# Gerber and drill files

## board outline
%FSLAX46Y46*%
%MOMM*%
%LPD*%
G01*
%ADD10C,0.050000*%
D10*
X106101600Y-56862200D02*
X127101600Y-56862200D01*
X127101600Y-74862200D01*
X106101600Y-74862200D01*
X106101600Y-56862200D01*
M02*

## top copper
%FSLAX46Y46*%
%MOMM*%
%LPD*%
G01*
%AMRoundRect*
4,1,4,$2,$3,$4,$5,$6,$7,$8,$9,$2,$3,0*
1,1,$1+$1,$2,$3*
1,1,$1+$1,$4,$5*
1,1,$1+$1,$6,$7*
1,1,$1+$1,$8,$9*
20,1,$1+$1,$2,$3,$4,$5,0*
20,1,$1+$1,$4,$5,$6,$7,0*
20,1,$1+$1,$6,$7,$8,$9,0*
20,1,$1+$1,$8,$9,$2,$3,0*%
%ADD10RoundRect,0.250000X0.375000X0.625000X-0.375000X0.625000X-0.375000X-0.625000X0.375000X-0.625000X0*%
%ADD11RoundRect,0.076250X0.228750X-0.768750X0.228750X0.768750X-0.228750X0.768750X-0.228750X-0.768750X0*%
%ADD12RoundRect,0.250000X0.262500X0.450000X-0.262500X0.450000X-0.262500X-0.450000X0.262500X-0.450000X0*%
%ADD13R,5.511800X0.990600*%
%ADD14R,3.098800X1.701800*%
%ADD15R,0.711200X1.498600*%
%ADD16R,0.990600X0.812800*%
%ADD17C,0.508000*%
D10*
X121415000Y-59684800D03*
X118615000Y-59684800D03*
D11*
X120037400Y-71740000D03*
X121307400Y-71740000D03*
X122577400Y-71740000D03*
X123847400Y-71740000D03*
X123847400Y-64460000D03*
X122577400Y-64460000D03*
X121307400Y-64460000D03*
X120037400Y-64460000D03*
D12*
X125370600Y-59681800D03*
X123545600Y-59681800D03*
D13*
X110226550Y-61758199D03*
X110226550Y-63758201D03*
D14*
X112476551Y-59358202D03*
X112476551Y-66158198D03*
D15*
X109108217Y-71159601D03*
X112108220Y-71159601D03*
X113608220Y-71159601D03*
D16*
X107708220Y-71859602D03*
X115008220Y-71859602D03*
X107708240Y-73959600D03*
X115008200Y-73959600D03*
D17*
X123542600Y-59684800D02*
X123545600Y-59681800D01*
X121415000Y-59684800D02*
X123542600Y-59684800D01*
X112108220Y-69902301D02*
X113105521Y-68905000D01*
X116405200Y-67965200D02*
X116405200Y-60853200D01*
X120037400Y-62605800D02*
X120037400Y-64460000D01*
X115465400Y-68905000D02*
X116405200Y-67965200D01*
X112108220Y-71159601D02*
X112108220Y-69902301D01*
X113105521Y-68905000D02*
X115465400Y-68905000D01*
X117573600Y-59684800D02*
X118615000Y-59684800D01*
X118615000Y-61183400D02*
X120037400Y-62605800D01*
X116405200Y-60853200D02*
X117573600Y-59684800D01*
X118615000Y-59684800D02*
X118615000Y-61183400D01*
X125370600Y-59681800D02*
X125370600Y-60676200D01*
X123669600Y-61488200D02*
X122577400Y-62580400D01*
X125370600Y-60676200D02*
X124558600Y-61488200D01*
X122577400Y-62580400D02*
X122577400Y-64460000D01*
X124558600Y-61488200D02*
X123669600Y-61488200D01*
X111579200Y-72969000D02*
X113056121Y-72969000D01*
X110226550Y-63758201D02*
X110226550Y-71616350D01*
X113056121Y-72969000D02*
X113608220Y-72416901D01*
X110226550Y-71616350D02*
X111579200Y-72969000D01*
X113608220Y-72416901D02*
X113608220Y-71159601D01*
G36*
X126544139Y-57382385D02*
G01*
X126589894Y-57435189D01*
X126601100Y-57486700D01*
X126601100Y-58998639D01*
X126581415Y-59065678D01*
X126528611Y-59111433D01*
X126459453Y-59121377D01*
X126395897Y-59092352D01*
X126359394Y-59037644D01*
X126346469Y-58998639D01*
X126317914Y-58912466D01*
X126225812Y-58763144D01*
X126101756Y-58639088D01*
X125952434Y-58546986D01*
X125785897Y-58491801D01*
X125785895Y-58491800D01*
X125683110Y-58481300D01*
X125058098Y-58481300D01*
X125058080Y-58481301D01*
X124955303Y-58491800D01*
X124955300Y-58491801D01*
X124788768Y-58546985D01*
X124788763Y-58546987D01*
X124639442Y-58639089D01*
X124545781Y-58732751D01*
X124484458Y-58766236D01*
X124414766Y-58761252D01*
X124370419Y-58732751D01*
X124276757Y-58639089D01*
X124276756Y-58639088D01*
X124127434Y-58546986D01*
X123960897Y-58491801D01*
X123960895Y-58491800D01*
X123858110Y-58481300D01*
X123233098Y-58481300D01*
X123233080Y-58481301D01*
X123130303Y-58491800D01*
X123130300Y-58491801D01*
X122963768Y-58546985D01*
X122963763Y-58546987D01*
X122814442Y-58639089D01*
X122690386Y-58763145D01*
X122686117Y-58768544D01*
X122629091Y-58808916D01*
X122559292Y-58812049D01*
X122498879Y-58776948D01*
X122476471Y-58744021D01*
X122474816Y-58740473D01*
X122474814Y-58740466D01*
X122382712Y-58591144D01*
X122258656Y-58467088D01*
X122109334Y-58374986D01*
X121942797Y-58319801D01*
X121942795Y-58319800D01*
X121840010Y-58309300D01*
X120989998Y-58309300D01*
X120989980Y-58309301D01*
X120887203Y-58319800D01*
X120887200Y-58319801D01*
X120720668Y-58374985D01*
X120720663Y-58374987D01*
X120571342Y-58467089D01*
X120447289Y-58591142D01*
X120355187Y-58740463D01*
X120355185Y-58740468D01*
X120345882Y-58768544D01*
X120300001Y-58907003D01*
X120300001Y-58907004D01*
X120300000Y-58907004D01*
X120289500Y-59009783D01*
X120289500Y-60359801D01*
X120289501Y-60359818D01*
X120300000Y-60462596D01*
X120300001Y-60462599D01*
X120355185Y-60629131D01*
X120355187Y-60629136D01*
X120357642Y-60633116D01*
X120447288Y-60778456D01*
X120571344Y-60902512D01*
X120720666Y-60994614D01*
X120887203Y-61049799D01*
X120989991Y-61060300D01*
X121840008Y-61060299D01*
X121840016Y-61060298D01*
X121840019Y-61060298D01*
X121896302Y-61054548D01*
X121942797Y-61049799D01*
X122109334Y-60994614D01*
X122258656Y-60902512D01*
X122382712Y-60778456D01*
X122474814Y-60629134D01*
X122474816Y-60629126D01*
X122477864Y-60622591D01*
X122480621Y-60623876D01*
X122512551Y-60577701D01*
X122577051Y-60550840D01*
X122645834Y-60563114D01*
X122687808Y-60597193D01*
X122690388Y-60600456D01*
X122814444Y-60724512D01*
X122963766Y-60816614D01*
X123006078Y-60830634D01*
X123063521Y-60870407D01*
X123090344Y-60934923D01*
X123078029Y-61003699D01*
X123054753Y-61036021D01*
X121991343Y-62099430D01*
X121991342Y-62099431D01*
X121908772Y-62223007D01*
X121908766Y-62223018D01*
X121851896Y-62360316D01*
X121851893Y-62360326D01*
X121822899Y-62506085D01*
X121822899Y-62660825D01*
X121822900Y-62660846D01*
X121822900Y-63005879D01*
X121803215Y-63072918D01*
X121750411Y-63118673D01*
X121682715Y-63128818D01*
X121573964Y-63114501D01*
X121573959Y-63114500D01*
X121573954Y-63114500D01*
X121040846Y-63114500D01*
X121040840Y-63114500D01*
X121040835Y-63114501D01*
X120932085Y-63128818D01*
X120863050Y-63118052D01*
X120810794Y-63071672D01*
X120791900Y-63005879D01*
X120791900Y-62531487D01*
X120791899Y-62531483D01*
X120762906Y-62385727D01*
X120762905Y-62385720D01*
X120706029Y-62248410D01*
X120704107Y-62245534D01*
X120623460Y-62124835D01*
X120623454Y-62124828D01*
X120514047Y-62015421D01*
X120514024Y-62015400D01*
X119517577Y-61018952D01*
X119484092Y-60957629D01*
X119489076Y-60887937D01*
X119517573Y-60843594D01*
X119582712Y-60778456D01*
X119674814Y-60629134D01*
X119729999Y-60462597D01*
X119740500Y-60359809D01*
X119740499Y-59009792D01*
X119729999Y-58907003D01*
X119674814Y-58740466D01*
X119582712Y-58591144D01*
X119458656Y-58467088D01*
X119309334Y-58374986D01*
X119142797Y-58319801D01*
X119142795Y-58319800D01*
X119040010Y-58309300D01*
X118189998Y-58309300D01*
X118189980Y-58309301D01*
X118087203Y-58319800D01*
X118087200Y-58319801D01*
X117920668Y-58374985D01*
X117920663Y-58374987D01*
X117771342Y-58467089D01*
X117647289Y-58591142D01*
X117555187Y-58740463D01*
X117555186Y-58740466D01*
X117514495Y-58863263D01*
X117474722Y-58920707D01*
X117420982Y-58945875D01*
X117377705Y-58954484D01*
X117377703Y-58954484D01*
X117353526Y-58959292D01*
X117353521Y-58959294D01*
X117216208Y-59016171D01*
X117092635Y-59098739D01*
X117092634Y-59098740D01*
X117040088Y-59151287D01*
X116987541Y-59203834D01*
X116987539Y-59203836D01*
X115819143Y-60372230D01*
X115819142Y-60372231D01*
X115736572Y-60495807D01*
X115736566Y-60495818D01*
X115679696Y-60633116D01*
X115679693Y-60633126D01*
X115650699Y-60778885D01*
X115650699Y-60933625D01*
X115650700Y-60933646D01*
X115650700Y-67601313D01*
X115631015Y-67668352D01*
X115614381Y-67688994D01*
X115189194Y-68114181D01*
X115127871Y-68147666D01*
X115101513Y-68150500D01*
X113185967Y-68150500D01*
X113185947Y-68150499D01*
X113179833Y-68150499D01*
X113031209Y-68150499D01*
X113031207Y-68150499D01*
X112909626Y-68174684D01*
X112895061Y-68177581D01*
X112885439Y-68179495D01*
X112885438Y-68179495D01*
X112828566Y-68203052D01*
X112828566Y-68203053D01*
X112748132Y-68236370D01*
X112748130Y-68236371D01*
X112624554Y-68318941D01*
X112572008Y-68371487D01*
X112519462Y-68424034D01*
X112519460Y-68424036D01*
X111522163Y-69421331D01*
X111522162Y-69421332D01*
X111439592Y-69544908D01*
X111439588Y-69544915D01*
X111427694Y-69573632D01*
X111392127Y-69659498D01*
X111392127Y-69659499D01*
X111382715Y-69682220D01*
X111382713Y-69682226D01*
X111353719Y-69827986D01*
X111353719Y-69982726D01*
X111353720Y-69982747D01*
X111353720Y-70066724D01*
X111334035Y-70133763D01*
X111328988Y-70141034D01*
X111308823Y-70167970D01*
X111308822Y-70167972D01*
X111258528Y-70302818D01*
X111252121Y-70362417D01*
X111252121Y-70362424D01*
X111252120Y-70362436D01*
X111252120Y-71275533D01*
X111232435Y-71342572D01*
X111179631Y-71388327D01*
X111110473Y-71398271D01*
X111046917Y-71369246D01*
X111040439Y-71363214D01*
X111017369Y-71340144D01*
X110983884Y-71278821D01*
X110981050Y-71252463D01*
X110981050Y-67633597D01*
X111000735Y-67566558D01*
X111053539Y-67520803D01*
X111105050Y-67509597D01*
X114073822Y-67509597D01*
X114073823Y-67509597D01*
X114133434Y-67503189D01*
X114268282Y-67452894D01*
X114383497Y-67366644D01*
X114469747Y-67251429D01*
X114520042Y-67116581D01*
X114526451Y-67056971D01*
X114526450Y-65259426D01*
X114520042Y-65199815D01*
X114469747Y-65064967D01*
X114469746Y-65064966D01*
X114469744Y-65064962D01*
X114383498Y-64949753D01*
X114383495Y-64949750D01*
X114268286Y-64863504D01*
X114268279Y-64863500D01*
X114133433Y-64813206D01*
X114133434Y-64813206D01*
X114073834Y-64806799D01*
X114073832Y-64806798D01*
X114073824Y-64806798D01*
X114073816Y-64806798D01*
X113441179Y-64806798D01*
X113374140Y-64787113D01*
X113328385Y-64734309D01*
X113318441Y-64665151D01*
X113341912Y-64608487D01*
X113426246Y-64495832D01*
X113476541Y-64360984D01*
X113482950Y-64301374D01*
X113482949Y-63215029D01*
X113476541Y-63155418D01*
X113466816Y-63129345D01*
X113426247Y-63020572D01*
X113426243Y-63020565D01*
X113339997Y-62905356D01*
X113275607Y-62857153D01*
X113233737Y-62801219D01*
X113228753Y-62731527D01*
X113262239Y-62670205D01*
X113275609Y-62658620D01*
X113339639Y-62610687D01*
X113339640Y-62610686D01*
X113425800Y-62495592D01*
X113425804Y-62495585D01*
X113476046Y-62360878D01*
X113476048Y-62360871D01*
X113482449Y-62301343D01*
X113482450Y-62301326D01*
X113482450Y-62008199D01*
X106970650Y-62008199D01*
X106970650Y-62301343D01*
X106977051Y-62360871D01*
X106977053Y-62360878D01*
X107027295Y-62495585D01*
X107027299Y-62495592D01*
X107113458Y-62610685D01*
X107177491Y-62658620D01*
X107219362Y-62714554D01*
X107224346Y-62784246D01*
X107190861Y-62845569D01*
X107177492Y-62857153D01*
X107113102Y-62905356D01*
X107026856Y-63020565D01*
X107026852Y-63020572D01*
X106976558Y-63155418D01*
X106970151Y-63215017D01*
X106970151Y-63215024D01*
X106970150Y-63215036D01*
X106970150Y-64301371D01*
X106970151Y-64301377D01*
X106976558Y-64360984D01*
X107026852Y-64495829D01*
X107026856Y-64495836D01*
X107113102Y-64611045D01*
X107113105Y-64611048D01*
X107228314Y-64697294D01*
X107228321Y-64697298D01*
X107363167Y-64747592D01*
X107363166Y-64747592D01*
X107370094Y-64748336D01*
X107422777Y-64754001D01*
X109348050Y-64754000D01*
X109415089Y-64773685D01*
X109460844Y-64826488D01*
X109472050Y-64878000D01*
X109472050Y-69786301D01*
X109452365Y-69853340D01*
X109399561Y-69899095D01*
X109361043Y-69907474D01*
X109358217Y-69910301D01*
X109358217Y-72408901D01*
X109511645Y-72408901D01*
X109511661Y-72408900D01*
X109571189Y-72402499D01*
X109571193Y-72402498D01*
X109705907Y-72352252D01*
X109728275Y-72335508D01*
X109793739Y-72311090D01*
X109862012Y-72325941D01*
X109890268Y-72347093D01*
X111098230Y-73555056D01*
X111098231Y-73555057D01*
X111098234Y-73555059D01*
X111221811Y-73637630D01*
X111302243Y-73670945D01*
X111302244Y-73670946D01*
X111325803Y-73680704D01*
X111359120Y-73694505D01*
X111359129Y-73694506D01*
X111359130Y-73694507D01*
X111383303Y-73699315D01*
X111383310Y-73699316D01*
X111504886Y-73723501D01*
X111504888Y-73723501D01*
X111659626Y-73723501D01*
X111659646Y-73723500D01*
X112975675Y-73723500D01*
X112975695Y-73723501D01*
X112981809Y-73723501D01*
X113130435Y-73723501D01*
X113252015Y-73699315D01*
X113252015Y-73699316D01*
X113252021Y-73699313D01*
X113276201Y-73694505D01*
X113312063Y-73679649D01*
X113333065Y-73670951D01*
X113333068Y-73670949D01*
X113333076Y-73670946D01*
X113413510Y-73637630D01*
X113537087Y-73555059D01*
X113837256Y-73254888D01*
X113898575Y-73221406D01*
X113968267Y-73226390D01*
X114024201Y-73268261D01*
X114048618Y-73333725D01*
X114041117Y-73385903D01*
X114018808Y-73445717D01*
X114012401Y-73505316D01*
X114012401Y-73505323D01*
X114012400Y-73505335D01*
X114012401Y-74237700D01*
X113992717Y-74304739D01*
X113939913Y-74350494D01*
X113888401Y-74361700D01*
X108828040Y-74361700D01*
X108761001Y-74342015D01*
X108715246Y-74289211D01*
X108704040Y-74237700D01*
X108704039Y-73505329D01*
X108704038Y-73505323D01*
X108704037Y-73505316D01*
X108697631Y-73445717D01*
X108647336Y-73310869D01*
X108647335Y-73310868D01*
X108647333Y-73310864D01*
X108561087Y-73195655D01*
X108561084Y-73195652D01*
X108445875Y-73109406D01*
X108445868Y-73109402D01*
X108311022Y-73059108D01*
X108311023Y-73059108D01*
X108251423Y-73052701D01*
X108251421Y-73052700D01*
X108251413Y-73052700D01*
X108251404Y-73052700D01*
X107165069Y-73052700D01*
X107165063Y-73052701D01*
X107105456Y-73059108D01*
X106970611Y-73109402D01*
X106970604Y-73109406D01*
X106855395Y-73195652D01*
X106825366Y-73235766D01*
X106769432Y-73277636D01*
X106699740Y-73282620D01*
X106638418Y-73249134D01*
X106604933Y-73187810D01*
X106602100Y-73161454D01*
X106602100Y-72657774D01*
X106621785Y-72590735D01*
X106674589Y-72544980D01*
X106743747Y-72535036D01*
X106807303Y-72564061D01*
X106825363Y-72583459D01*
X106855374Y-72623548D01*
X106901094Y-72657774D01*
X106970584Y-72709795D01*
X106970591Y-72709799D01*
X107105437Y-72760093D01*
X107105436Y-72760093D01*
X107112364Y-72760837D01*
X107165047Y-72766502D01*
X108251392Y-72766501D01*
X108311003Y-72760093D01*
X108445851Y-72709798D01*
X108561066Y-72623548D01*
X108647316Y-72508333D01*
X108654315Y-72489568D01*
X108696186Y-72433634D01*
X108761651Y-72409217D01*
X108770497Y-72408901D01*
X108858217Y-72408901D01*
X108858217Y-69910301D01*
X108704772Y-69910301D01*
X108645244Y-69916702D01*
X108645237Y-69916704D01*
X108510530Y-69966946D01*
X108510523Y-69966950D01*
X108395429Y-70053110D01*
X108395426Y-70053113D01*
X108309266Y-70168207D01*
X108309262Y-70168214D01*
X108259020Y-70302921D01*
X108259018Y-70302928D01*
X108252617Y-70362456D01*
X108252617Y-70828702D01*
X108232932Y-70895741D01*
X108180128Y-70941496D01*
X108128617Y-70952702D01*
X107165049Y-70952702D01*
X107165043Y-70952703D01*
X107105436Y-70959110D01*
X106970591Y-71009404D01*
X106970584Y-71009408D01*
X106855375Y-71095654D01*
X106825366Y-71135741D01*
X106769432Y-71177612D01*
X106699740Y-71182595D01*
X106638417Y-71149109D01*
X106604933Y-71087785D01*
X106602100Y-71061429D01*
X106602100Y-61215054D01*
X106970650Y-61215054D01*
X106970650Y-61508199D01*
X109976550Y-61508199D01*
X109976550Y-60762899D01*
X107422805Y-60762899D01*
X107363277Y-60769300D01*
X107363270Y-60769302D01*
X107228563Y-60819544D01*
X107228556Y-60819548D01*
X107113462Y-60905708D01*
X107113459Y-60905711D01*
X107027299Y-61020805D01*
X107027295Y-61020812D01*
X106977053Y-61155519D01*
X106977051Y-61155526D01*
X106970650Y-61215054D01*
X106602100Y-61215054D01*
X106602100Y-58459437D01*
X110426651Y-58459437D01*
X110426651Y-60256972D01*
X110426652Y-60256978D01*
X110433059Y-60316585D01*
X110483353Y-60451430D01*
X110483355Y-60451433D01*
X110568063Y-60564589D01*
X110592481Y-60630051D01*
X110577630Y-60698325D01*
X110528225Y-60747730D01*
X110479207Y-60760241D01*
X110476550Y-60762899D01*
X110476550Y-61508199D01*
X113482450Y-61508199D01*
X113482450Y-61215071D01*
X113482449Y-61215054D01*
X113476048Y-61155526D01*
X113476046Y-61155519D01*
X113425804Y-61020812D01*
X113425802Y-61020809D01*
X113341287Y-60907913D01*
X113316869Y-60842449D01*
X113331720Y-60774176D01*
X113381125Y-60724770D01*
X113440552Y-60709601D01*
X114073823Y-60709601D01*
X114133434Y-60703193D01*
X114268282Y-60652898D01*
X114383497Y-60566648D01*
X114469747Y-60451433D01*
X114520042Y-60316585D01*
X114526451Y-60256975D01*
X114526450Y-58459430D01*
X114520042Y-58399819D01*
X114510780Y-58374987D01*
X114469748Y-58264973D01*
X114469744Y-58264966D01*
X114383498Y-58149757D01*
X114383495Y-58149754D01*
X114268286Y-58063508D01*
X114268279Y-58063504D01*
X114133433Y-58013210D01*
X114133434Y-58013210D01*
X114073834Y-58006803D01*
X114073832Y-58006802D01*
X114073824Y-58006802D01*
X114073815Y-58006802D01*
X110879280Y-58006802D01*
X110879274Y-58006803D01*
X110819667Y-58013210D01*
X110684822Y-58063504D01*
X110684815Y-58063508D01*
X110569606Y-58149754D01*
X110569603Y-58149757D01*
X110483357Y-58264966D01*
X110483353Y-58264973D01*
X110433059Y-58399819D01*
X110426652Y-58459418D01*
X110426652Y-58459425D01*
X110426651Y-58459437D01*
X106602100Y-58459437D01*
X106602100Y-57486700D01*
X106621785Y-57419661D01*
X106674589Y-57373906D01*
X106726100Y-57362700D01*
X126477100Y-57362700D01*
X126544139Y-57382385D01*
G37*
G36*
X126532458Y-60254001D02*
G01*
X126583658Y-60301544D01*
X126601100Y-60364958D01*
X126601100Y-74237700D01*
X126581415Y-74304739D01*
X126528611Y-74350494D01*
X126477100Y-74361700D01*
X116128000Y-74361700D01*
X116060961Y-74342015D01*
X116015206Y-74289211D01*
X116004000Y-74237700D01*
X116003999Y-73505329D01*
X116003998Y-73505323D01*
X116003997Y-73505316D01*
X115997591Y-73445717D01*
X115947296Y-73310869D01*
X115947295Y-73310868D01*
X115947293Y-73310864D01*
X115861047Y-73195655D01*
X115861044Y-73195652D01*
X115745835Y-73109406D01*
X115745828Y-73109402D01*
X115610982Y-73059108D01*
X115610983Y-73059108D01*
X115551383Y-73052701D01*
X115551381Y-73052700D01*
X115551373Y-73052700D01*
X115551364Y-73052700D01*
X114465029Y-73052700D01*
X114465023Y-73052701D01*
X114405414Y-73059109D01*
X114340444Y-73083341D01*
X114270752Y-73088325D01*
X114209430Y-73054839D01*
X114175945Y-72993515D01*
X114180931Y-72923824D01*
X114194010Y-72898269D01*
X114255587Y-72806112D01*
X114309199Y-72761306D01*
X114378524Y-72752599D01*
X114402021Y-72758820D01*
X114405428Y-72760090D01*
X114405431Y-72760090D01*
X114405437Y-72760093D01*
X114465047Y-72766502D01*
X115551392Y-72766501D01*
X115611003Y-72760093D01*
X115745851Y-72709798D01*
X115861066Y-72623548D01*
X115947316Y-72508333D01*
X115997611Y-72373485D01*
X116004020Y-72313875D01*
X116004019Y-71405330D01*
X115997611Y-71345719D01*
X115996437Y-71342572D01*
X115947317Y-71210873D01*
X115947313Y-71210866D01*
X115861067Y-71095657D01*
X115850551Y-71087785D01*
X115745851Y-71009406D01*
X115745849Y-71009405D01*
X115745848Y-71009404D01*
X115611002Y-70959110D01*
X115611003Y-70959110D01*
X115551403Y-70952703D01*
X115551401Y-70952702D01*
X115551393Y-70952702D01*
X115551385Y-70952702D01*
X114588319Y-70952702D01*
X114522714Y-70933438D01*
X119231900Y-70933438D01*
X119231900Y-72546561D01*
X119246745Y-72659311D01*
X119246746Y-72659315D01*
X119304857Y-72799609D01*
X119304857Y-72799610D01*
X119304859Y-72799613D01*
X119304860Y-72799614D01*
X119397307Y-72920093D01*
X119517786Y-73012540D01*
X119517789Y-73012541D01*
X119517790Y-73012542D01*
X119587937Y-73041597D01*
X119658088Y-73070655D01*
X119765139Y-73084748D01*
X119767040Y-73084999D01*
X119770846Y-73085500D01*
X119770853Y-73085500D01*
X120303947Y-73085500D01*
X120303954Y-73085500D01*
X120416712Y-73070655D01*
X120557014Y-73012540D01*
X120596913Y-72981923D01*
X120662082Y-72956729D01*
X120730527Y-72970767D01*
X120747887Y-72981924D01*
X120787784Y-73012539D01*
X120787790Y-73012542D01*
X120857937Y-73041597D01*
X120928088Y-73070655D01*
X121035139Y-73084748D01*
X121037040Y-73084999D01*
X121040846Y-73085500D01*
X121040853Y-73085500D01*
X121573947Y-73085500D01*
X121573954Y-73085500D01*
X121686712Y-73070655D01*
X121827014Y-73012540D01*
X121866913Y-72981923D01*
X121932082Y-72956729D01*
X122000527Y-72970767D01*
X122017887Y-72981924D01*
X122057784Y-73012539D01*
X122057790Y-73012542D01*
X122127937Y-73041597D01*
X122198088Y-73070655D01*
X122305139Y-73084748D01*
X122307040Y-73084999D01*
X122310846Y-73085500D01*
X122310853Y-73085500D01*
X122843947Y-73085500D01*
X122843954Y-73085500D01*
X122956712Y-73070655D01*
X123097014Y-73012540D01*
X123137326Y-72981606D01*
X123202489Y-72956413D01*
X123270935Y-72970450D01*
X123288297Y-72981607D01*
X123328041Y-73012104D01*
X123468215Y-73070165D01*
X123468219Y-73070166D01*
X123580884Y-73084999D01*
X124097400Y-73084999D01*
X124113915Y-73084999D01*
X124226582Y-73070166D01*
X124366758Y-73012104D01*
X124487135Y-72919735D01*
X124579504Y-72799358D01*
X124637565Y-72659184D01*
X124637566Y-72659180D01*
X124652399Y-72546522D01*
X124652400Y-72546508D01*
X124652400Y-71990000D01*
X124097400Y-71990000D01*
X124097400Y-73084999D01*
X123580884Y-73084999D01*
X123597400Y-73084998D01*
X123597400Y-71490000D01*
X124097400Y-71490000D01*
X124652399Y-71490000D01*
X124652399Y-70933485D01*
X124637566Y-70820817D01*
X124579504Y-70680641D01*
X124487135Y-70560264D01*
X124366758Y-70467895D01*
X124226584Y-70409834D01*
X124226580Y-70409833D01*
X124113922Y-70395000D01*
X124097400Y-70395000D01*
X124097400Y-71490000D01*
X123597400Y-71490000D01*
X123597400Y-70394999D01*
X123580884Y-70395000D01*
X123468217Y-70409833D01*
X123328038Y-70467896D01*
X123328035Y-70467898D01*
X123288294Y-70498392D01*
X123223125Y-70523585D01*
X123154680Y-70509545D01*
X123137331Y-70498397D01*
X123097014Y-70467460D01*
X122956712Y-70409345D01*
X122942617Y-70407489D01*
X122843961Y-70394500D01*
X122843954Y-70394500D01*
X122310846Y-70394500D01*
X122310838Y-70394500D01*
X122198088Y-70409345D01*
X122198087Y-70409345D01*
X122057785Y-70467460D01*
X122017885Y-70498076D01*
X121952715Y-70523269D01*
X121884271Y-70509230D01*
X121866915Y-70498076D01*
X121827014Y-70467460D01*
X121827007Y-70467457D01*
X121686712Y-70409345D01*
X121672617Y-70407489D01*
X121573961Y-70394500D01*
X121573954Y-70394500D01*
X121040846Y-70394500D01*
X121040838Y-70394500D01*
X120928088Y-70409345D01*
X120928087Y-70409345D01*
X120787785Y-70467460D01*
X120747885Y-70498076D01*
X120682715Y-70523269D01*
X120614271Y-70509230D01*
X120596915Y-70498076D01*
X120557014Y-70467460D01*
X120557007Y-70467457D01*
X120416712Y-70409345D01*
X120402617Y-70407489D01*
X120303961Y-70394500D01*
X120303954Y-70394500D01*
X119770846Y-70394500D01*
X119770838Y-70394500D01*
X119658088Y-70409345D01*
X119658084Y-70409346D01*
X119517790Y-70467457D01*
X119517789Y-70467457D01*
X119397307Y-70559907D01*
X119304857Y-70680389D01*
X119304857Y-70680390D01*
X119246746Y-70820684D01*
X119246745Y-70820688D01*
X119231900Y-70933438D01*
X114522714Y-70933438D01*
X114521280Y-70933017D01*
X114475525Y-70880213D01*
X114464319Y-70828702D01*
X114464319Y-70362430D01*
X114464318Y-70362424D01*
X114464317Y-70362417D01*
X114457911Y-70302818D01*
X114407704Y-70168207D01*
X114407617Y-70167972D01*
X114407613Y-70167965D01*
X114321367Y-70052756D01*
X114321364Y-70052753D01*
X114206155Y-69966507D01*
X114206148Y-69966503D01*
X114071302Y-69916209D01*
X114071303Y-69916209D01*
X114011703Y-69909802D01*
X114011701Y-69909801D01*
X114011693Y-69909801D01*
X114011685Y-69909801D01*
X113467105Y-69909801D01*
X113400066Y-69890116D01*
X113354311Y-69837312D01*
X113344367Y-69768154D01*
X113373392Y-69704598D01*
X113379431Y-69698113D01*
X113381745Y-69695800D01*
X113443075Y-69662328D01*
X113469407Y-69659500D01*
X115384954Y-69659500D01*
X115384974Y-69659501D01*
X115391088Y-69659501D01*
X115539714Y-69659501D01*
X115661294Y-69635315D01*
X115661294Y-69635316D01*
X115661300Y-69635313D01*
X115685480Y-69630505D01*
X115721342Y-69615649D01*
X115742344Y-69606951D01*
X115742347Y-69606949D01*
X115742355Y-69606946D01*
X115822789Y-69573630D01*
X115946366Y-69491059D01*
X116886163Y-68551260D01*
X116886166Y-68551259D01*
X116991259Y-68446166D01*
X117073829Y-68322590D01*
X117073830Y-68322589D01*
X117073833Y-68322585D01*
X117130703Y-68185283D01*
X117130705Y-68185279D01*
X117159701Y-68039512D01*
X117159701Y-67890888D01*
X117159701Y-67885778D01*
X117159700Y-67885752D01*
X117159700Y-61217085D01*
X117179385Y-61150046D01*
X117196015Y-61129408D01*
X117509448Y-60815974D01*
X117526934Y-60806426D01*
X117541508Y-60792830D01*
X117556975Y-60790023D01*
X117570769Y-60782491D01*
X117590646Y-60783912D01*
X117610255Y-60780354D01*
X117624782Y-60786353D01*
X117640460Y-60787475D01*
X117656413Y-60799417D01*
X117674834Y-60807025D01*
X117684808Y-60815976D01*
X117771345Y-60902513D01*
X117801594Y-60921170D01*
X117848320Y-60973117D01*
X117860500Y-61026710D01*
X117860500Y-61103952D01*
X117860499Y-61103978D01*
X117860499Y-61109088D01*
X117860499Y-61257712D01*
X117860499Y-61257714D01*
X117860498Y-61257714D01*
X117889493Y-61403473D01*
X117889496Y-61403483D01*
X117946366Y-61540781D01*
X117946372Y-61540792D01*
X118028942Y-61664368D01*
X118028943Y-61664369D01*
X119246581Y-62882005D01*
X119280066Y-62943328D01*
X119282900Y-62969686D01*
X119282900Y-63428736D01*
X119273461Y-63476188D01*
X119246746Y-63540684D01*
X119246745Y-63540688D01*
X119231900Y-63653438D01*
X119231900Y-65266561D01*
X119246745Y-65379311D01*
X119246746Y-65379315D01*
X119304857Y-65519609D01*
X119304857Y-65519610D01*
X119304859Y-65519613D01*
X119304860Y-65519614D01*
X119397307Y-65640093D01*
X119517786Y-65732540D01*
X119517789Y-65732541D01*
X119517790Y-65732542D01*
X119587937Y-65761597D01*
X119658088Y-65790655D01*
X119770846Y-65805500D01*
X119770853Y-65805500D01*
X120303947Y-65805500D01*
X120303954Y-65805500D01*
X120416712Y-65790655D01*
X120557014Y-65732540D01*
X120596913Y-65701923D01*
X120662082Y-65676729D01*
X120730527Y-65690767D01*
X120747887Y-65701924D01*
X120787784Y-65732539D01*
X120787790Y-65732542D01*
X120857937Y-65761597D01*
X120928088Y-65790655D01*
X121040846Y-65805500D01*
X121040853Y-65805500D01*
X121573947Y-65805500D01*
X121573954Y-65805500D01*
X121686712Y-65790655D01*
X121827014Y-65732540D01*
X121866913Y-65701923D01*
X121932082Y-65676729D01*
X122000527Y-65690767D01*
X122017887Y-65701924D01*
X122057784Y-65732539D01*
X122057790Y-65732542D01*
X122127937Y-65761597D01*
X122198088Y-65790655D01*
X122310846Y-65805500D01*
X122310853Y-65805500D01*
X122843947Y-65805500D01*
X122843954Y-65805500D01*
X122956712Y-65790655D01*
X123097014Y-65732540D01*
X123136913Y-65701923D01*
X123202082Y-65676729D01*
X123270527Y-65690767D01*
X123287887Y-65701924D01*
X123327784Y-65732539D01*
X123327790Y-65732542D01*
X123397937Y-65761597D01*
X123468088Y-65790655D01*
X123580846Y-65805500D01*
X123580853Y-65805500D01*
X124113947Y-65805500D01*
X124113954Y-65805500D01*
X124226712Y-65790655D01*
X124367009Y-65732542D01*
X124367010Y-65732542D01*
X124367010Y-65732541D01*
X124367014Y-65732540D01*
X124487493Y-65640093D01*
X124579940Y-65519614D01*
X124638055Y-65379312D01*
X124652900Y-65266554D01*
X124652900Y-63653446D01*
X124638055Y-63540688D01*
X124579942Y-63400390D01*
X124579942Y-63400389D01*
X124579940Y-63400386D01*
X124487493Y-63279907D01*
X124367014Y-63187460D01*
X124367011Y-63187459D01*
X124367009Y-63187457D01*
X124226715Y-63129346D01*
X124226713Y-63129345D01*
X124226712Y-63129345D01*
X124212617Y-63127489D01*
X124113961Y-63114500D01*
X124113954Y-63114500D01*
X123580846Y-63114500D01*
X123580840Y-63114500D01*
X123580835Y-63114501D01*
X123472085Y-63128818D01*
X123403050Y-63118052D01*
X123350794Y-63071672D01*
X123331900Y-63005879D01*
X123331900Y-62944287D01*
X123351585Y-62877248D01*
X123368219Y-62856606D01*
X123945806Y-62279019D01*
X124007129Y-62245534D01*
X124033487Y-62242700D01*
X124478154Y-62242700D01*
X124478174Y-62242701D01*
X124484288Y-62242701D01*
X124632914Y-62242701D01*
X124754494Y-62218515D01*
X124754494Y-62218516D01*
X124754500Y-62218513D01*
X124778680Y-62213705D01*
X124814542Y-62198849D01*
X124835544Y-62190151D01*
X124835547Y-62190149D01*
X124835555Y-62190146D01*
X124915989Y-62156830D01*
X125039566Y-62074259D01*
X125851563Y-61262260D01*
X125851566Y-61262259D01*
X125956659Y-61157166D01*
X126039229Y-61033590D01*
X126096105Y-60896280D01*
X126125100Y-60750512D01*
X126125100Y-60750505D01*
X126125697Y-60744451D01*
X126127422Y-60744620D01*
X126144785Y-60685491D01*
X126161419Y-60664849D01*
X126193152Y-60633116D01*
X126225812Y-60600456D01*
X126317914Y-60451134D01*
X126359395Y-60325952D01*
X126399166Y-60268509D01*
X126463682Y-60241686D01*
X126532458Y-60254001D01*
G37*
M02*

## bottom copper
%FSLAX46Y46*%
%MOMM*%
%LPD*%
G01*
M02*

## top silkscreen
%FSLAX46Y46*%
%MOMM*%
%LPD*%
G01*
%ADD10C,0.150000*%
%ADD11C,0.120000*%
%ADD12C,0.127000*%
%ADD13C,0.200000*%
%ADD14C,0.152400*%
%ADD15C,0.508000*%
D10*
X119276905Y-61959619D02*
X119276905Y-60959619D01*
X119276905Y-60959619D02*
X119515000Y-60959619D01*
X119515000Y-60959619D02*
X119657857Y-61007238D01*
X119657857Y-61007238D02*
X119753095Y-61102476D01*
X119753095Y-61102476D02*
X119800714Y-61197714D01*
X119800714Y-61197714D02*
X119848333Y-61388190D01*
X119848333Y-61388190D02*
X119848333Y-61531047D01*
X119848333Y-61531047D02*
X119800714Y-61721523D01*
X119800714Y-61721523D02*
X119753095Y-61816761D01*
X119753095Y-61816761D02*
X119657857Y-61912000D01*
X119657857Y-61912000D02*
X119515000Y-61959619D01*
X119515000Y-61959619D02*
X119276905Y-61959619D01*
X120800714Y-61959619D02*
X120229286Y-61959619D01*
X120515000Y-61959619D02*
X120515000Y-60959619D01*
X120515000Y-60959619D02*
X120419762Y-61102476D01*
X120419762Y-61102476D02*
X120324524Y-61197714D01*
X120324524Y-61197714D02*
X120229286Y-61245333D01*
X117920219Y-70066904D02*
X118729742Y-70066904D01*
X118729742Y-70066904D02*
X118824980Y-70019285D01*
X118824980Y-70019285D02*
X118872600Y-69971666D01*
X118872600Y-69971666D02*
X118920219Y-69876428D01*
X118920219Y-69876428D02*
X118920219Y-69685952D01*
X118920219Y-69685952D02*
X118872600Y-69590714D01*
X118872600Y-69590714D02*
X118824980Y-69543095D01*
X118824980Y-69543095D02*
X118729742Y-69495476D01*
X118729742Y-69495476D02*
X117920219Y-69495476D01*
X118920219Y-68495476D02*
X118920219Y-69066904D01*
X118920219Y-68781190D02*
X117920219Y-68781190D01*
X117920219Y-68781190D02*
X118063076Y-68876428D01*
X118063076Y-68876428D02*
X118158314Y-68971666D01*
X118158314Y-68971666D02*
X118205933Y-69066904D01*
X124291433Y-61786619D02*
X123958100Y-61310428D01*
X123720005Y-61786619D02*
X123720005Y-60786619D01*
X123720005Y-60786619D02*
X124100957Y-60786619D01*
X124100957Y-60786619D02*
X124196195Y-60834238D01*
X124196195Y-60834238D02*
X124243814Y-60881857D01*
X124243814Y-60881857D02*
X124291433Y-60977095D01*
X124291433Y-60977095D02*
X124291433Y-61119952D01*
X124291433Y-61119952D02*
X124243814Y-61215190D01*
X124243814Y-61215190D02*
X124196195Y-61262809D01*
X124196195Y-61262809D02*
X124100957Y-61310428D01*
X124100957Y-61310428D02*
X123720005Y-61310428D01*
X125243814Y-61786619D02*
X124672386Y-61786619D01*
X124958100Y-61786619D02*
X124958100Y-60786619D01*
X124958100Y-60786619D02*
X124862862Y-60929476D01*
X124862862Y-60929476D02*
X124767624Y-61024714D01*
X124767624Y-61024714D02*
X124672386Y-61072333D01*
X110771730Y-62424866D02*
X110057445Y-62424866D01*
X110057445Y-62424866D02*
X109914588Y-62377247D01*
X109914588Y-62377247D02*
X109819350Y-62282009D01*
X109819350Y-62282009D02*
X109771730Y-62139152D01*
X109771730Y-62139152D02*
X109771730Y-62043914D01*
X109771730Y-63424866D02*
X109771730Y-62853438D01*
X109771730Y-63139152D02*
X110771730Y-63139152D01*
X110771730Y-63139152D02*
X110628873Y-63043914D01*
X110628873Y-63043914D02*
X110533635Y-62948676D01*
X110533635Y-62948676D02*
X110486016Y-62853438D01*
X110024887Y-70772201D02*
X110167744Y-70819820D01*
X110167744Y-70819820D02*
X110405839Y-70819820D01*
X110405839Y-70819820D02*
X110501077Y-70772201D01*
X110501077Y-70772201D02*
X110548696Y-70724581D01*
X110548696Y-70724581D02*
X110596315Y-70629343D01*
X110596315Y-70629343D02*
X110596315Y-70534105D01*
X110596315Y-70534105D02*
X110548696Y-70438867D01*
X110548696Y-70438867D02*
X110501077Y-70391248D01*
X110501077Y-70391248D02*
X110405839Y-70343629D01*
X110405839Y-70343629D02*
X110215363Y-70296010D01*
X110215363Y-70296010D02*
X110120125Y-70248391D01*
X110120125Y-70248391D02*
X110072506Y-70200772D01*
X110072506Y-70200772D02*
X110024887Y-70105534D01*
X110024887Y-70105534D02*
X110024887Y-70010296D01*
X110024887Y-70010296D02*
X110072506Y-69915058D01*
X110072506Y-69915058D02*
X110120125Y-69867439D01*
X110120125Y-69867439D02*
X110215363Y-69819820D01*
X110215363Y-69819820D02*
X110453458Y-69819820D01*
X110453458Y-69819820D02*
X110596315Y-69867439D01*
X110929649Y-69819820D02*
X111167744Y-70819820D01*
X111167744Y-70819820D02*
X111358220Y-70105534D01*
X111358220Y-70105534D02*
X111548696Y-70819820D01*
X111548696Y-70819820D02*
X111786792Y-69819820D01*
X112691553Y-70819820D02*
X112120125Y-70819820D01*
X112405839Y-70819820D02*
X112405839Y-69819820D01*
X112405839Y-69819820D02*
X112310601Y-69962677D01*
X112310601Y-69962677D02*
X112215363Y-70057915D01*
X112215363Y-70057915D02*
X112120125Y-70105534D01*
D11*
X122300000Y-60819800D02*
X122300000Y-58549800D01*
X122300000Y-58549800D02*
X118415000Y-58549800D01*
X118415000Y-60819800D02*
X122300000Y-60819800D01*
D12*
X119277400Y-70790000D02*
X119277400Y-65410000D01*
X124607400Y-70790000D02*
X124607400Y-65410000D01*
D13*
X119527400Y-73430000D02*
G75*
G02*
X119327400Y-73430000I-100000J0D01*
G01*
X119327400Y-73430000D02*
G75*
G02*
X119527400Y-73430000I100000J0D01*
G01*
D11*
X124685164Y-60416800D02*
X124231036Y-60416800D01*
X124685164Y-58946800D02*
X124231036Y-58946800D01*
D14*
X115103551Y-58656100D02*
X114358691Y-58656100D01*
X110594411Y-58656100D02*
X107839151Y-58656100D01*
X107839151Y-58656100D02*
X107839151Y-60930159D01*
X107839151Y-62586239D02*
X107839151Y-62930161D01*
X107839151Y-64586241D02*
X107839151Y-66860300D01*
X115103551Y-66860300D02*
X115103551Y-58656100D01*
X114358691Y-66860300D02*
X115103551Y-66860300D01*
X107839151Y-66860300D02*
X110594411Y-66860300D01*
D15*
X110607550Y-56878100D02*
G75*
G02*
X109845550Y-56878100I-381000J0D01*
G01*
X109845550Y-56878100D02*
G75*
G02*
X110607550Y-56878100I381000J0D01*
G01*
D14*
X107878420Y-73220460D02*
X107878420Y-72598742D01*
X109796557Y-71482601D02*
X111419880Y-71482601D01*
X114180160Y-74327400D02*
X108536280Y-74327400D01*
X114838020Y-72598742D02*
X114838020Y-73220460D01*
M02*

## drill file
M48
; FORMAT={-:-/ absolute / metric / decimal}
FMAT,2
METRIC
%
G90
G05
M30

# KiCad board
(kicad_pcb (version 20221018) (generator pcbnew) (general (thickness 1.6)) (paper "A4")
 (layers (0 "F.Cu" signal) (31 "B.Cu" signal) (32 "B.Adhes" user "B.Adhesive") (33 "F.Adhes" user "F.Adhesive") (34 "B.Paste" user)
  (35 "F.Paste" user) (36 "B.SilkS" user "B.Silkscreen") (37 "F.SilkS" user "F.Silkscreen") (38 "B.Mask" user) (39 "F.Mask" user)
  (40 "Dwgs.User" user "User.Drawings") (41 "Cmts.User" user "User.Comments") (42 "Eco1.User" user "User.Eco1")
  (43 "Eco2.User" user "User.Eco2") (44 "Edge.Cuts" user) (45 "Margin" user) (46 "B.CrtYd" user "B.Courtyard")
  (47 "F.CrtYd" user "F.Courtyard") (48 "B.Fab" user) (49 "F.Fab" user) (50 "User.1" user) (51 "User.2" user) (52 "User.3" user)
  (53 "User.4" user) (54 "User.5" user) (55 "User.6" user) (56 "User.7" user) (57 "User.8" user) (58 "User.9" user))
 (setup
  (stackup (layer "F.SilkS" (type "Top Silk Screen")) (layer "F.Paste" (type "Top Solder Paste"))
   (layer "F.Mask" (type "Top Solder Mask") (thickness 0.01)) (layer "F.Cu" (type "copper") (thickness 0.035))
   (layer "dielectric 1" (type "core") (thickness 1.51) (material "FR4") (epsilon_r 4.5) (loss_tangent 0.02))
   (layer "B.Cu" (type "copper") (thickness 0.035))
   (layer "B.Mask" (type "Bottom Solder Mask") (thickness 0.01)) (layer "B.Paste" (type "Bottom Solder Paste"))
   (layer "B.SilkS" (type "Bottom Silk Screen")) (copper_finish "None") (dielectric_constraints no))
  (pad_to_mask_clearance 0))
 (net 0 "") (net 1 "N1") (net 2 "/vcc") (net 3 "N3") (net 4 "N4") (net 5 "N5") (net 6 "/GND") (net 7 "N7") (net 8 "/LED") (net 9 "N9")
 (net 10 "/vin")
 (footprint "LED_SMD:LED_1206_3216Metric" (layer "F.Cu") (at 120.015 59.6848 180)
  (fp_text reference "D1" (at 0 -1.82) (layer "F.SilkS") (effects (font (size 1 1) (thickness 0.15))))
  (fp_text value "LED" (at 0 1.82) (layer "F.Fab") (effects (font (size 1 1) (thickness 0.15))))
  (fp_line (start -2.285 -1.135) (end -2.285 1.135) (stroke (width 0.12) (type solid)) (layer "F.SilkS"))
  (fp_line (start -2.285 1.135) (end 1.6 1.135) (stroke (width 0.12) (type solid)) (layer "F.SilkS"))
  (fp_line (start 1.6 -1.135) (end -2.285 -1.135) (stroke (width 0.12) (type solid)) (layer "F.SilkS"))
  (pad "1" smd roundrect (at -1.4 0 180) (size 1.25 1.75) (layers "F.Cu" "F.Paste" "F.Mask") (roundrect_rratio 0.2) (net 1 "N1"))
  (pad "2" smd roundrect (at 1.4 0 180) (size 1.25 1.75) (layers "F.Cu" "F.Paste" "F.Mask") (roundrect_rratio 0.2) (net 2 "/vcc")))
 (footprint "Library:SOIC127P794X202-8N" (layer "F.Cu") (at 121.9424 68.1 90)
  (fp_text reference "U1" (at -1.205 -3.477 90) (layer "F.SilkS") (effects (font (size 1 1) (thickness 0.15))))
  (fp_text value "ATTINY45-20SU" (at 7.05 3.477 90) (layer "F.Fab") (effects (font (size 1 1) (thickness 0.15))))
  (fp_line (start -2.69 -2.665) (end 2.69 -2.665) (stroke (width 0.127) (type solid)) (layer "F.SilkS"))
  (fp_line (start -2.69 2.665) (end 2.69 2.665) (stroke (width 0.127) (type solid)) (layer "F.SilkS"))
  (fp_circle (center -5.33 -2.515) (end -5.23 -2.515) (stroke (width 0.2) (type solid)) (fill none) (layer "F.SilkS"))
  (pad "1" smd roundrect (at -3.64 -1.905 90) (size 1.69 0.61) (layers "F.Cu" "F.Paste" "F.Mask") (roundrect_rratio 0.125) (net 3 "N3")
   (solder_mask_margin 0.102))
  (pad "2" smd roundrect (at -3.64 -0.635 90) (size 1.69 0.61) (layers "F.Cu" "F.Paste" "F.Mask") (roundrect_rratio 0.125) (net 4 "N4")
   (solder_mask_margin 0.102))
  (pad "3" smd roundrect (at -3.64 0.635 90) (size 1.69 0.61) (layers "F.Cu" "F.Paste" "F.Mask") (roundrect_rratio 0.125) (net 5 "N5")
   (solder_mask_margin 0.102))
  (pad "4" smd roundrect (at -3.64 1.905 90) (size 1.69 0.61) (layers "F.Cu" "F.Paste" "F.Mask") (roundrect_rratio 0.125) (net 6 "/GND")
   (solder_mask_margin 0.102))
  (pad "5" smd roundrect (at 3.64 1.905 90) (size 1.69 0.61) (layers "F.Cu" "F.Paste" "F.Mask") (roundrect_rratio 0.125) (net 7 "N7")
   (solder_mask_margin 0.102))
  (pad "6" smd roundrect (at 3.64 0.635 90) (size 1.69 0.61) (layers "F.Cu" "F.Paste" "F.Mask") (roundrect_rratio 0.125) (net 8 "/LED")
   (solder_mask_margin 0.102))
  (pad "7" smd roundrect (at 3.64 -0.635 90) (size 1.69 0.61) (layers "F.Cu" "F.Paste" "F.Mask") (roundrect_rratio 0.125) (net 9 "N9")
   (solder_mask_margin 0.102))
  (pad "8" smd roundrect (at 3.64 -1.905 90) (size 1.69 0.61) (layers "F.Cu" "F.Paste" "F.Mask") (roundrect_rratio 0.125) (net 2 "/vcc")
   (solder_mask_margin 0.102)))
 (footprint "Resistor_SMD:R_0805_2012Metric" (layer "F.Cu") (at 124.4581 59.6818 180)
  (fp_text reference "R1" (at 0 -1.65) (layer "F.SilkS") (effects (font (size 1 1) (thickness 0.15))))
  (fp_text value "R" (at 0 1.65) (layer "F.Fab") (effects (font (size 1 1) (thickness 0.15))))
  (fp_line (start -0.227064 -0.735) (end 0.227064 -0.735) (stroke (width 0.12) (type solid)) (layer "F.SilkS"))
  (fp_line (start -0.227064 0.735) (end 0.227064 0.735) (stroke (width 0.12) (type solid)) (layer "F.SilkS"))
  (pad "1" smd roundrect (at -0.9125 0 180) (size 1.025 1.4) (layers "F.Cu" "F.Paste" "F.Mask") (roundrect_rratio 0.243902439)
   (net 8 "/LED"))
  (pad "2" smd roundrect (at 0.9125 0 180) (size 1.025 1.4) (layers "F.Cu" "F.Paste" "F.Mask") (roundrect_rratio 0.243902439) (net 1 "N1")))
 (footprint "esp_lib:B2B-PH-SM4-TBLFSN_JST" (layer "F.Cu") (at 111.471351 62.7582 -90)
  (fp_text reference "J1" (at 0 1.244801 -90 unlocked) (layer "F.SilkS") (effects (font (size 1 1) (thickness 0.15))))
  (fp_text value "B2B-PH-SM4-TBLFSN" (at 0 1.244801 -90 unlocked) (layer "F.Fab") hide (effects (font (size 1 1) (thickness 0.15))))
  (fp_line (start -4.1021 -3.6322) (end -4.1021 -2.88734) (stroke (width 0.1524) (type solid)) (layer "F.SilkS"))
  (fp_line (start -4.1021 0.87694) (end -4.1021 3.6322) (stroke (width 0.1524) (type solid)) (layer "F.SilkS"))
  (fp_line (start -4.1021 3.6322) (end -1.828041 3.6322) (stroke (width 0.1524) (type solid)) (layer "F.SilkS"))
  (fp_line (start -0.171961 3.6322) (end 0.171961 3.6322) (stroke (width 0.1524) (type solid)) (layer "F.SilkS"))
  (fp_line (start 1.828041 3.6322) (end 4.1021 3.6322) (stroke (width 0.1524) (type solid)) (layer "F.SilkS"))
  (fp_line (start 4.1021 -3.6322) (end -4.1021 -3.6322) (stroke (width 0.1524) (type solid)) (layer "F.SilkS"))
  (fp_line (start 4.1021 -2.88734) (end 4.1021 -3.6322) (stroke (width 0.1524) (type solid)) (layer "F.SilkS"))
  (fp_line (start 4.1021 3.6322) (end 4.1021 0.87694) (stroke (width 0.1524) (type solid)) (layer "F.SilkS"))
  (fp_circle (center -5.8801 1.244801) (end -5.4991 1.244801) (stroke (width 0.508) (type solid)) (fill none) (layer "F.SilkS"))
  (pad "1" smd rect (at -1.000001 1.244801 270) (size 0.9906 5.5118) (layers "F.Cu" "F.Paste" "F.Mask") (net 6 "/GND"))
  (pad "2" smd rect (at 1.000001 1.244801 270) (size 0.9906 5.5118) (layers "F.Cu" "F.Paste" "F.Mask") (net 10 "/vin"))
  (pad "3" smd rect (at -3.399998 -1.0052) (size 3.0988 1.7018) (layers "F.Cu" "F.Paste" "F.Mask"))
  (pad "4" smd rect (at 3.399998 -1.0052) (size 3.0988 1.7018) (layers "F.Cu" "F.Paste" "F.Mask")))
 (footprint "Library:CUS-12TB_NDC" (layer "F.Cu") (at 111.35822 72.905001)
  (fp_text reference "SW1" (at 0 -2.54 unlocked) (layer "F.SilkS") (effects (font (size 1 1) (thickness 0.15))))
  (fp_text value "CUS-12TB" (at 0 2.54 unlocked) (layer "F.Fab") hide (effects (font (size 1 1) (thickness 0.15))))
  (fp_line (start -3.4798 0.315459) (end -3.4798 -0.306259) (stroke (width 0.1524) (type solid)) (layer "F.SilkS"))
  (fp_line (start -1.561663 -1.4224) (end 0.06166 -1.4224) (stroke (width 0.1524) (type solid)) (layer "F.SilkS"))
  (fp_line (start 2.82194 1.422399) (end -2.82194 1.422399) (stroke (width 0.1524) (type solid)) (layer "F.SilkS"))
  (fp_line (start 3.4798 -0.306259) (end 3.4798 0.315459) (stroke (width 0.1524) (type solid)) (layer "F.SilkS"))
  (pad "1" smd rect (at -2.250003 -1.7454) (size 0.7112 1.4986) (layers "F.Cu" "F.Paste" "F.Mask") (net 6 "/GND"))
  (pad "2" smd rect (at 0.75 -1.7454) (size 0.7112 1.4986) (layers "F.Cu" "F.Paste" "F.Mask") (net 2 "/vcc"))
  (pad "3" smd rect (at 2.25 -1.7454) (size 0.7112 1.4986) (layers "F.Cu" "F.Paste" "F.Mask") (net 10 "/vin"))
  (pad "4" smd rect (at -3.65 -1.045399) (size 0.9906 0.8128) (layers "F.Cu" "F.Paste" "F.Mask"))
  (pad "5" smd rect (at 3.65 -1.045399) (size 0.9906 0.8128) (layers "F.Cu" "F.Paste" "F.Mask"))
  (pad "6" smd rect (at -3.64998 1.054599) (size 0.9906 0.8128) (layers "F.Cu" "F.Paste" "F.Mask"))
  (pad "7" smd rect (at 3.64998 1.054599) (size 0.9906 0.8128) (layers "F.Cu" "F.Paste" "F.Mask")))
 (gr_rect (start 106.1016 56.8622) (end 127.1016 74.8622) (stroke (width 0.05) (type default)) (fill none) (layer "Edge.Cuts"))
 (segment (start 123.5426 59.6848) (end 123.5456 59.6818) (width 0.508) (layer "F.Cu") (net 1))
 (segment (start 121.415 59.6848) (end 123.5426 59.6848) (width 0.508) (layer "F.Cu") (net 1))
 (segment (start 112.10822 69.902301) (end 113.105521 68.905) (width 0.508) (layer "F.Cu") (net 2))
 (segment (start 116.4052 67.9652) (end 116.4052 60.8532) (width 0.508) (layer "F.Cu") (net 2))
 (segment (start 120.0374 62.6058) (end 120.0374 64.46) (width 0.508) (layer "F.Cu") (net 2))
 (segment (start 115.4654 68.905) (end 116.4052 67.9652) (width 0.508) (layer "F.Cu") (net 2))
 (segment (start 112.10822 71.159601) (end 112.10822 69.902301) (width 0.508) (layer "F.Cu") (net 2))
 (segment (start 113.105521 68.905) (end 115.4654 68.905) (width 0.508) (layer "F.Cu") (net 2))
 (segment (start 117.5736 59.6848) (end 118.615 59.6848) (width 0.508) (layer "F.Cu") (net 2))
 (segment (start 118.615 61.1834) (end 120.0374 62.6058) (width 0.508) (layer "F.Cu") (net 2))
 (segment (start 116.4052 60.8532) (end 117.5736 59.6848) (width 0.508) (layer "F.Cu") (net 2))
 (segment (start 118.615 59.6848) (end 118.615 61.1834) (width 0.508) (layer "F.Cu") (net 2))
 (segment (start 125.3706 59.6818) (end 125.3706 60.6762) (width 0.508) (layer "F.Cu") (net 8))
 (segment (start 123.6696 61.4882) (end 122.5774 62.5804) (width 0.508) (layer "F.Cu") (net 8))
 (segment (start 125.3706 60.6762) (end 124.5586 61.4882) (width 0.508) (layer "F.Cu") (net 8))
 (segment (start 122.5774 62.5804) (end 122.5774 64.46) (width 0.508) (layer "F.Cu") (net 8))
 (segment (start 124.5586 61.4882) (end 123.6696 61.4882) (width 0.508) (layer "F.Cu") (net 8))
 (segment (start 111.5792 72.969) (end 113.056121 72.969) (width 0.508) (layer "F.Cu") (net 10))
 (segment (start 110.22655 63.758201) (end 110.22655 71.61635) (width 0.508) (layer "F.Cu") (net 10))
 (segment (start 113.056121 72.969) (end 113.60822 72.416901) (width 0.508) (layer "F.Cu") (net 10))
 (segment (start 110.22655 71.61635) (end 111.5792 72.969) (width 0.508) (layer "F.Cu") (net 10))
 (segment (start 113.60822 72.416901) (end 113.60822 71.159601) (width 0.508) (layer "F.Cu") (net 10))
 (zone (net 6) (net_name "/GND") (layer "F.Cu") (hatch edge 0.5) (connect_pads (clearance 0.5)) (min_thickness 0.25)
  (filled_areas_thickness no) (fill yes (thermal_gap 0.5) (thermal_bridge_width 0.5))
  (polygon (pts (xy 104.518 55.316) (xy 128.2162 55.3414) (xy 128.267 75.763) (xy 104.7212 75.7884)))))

